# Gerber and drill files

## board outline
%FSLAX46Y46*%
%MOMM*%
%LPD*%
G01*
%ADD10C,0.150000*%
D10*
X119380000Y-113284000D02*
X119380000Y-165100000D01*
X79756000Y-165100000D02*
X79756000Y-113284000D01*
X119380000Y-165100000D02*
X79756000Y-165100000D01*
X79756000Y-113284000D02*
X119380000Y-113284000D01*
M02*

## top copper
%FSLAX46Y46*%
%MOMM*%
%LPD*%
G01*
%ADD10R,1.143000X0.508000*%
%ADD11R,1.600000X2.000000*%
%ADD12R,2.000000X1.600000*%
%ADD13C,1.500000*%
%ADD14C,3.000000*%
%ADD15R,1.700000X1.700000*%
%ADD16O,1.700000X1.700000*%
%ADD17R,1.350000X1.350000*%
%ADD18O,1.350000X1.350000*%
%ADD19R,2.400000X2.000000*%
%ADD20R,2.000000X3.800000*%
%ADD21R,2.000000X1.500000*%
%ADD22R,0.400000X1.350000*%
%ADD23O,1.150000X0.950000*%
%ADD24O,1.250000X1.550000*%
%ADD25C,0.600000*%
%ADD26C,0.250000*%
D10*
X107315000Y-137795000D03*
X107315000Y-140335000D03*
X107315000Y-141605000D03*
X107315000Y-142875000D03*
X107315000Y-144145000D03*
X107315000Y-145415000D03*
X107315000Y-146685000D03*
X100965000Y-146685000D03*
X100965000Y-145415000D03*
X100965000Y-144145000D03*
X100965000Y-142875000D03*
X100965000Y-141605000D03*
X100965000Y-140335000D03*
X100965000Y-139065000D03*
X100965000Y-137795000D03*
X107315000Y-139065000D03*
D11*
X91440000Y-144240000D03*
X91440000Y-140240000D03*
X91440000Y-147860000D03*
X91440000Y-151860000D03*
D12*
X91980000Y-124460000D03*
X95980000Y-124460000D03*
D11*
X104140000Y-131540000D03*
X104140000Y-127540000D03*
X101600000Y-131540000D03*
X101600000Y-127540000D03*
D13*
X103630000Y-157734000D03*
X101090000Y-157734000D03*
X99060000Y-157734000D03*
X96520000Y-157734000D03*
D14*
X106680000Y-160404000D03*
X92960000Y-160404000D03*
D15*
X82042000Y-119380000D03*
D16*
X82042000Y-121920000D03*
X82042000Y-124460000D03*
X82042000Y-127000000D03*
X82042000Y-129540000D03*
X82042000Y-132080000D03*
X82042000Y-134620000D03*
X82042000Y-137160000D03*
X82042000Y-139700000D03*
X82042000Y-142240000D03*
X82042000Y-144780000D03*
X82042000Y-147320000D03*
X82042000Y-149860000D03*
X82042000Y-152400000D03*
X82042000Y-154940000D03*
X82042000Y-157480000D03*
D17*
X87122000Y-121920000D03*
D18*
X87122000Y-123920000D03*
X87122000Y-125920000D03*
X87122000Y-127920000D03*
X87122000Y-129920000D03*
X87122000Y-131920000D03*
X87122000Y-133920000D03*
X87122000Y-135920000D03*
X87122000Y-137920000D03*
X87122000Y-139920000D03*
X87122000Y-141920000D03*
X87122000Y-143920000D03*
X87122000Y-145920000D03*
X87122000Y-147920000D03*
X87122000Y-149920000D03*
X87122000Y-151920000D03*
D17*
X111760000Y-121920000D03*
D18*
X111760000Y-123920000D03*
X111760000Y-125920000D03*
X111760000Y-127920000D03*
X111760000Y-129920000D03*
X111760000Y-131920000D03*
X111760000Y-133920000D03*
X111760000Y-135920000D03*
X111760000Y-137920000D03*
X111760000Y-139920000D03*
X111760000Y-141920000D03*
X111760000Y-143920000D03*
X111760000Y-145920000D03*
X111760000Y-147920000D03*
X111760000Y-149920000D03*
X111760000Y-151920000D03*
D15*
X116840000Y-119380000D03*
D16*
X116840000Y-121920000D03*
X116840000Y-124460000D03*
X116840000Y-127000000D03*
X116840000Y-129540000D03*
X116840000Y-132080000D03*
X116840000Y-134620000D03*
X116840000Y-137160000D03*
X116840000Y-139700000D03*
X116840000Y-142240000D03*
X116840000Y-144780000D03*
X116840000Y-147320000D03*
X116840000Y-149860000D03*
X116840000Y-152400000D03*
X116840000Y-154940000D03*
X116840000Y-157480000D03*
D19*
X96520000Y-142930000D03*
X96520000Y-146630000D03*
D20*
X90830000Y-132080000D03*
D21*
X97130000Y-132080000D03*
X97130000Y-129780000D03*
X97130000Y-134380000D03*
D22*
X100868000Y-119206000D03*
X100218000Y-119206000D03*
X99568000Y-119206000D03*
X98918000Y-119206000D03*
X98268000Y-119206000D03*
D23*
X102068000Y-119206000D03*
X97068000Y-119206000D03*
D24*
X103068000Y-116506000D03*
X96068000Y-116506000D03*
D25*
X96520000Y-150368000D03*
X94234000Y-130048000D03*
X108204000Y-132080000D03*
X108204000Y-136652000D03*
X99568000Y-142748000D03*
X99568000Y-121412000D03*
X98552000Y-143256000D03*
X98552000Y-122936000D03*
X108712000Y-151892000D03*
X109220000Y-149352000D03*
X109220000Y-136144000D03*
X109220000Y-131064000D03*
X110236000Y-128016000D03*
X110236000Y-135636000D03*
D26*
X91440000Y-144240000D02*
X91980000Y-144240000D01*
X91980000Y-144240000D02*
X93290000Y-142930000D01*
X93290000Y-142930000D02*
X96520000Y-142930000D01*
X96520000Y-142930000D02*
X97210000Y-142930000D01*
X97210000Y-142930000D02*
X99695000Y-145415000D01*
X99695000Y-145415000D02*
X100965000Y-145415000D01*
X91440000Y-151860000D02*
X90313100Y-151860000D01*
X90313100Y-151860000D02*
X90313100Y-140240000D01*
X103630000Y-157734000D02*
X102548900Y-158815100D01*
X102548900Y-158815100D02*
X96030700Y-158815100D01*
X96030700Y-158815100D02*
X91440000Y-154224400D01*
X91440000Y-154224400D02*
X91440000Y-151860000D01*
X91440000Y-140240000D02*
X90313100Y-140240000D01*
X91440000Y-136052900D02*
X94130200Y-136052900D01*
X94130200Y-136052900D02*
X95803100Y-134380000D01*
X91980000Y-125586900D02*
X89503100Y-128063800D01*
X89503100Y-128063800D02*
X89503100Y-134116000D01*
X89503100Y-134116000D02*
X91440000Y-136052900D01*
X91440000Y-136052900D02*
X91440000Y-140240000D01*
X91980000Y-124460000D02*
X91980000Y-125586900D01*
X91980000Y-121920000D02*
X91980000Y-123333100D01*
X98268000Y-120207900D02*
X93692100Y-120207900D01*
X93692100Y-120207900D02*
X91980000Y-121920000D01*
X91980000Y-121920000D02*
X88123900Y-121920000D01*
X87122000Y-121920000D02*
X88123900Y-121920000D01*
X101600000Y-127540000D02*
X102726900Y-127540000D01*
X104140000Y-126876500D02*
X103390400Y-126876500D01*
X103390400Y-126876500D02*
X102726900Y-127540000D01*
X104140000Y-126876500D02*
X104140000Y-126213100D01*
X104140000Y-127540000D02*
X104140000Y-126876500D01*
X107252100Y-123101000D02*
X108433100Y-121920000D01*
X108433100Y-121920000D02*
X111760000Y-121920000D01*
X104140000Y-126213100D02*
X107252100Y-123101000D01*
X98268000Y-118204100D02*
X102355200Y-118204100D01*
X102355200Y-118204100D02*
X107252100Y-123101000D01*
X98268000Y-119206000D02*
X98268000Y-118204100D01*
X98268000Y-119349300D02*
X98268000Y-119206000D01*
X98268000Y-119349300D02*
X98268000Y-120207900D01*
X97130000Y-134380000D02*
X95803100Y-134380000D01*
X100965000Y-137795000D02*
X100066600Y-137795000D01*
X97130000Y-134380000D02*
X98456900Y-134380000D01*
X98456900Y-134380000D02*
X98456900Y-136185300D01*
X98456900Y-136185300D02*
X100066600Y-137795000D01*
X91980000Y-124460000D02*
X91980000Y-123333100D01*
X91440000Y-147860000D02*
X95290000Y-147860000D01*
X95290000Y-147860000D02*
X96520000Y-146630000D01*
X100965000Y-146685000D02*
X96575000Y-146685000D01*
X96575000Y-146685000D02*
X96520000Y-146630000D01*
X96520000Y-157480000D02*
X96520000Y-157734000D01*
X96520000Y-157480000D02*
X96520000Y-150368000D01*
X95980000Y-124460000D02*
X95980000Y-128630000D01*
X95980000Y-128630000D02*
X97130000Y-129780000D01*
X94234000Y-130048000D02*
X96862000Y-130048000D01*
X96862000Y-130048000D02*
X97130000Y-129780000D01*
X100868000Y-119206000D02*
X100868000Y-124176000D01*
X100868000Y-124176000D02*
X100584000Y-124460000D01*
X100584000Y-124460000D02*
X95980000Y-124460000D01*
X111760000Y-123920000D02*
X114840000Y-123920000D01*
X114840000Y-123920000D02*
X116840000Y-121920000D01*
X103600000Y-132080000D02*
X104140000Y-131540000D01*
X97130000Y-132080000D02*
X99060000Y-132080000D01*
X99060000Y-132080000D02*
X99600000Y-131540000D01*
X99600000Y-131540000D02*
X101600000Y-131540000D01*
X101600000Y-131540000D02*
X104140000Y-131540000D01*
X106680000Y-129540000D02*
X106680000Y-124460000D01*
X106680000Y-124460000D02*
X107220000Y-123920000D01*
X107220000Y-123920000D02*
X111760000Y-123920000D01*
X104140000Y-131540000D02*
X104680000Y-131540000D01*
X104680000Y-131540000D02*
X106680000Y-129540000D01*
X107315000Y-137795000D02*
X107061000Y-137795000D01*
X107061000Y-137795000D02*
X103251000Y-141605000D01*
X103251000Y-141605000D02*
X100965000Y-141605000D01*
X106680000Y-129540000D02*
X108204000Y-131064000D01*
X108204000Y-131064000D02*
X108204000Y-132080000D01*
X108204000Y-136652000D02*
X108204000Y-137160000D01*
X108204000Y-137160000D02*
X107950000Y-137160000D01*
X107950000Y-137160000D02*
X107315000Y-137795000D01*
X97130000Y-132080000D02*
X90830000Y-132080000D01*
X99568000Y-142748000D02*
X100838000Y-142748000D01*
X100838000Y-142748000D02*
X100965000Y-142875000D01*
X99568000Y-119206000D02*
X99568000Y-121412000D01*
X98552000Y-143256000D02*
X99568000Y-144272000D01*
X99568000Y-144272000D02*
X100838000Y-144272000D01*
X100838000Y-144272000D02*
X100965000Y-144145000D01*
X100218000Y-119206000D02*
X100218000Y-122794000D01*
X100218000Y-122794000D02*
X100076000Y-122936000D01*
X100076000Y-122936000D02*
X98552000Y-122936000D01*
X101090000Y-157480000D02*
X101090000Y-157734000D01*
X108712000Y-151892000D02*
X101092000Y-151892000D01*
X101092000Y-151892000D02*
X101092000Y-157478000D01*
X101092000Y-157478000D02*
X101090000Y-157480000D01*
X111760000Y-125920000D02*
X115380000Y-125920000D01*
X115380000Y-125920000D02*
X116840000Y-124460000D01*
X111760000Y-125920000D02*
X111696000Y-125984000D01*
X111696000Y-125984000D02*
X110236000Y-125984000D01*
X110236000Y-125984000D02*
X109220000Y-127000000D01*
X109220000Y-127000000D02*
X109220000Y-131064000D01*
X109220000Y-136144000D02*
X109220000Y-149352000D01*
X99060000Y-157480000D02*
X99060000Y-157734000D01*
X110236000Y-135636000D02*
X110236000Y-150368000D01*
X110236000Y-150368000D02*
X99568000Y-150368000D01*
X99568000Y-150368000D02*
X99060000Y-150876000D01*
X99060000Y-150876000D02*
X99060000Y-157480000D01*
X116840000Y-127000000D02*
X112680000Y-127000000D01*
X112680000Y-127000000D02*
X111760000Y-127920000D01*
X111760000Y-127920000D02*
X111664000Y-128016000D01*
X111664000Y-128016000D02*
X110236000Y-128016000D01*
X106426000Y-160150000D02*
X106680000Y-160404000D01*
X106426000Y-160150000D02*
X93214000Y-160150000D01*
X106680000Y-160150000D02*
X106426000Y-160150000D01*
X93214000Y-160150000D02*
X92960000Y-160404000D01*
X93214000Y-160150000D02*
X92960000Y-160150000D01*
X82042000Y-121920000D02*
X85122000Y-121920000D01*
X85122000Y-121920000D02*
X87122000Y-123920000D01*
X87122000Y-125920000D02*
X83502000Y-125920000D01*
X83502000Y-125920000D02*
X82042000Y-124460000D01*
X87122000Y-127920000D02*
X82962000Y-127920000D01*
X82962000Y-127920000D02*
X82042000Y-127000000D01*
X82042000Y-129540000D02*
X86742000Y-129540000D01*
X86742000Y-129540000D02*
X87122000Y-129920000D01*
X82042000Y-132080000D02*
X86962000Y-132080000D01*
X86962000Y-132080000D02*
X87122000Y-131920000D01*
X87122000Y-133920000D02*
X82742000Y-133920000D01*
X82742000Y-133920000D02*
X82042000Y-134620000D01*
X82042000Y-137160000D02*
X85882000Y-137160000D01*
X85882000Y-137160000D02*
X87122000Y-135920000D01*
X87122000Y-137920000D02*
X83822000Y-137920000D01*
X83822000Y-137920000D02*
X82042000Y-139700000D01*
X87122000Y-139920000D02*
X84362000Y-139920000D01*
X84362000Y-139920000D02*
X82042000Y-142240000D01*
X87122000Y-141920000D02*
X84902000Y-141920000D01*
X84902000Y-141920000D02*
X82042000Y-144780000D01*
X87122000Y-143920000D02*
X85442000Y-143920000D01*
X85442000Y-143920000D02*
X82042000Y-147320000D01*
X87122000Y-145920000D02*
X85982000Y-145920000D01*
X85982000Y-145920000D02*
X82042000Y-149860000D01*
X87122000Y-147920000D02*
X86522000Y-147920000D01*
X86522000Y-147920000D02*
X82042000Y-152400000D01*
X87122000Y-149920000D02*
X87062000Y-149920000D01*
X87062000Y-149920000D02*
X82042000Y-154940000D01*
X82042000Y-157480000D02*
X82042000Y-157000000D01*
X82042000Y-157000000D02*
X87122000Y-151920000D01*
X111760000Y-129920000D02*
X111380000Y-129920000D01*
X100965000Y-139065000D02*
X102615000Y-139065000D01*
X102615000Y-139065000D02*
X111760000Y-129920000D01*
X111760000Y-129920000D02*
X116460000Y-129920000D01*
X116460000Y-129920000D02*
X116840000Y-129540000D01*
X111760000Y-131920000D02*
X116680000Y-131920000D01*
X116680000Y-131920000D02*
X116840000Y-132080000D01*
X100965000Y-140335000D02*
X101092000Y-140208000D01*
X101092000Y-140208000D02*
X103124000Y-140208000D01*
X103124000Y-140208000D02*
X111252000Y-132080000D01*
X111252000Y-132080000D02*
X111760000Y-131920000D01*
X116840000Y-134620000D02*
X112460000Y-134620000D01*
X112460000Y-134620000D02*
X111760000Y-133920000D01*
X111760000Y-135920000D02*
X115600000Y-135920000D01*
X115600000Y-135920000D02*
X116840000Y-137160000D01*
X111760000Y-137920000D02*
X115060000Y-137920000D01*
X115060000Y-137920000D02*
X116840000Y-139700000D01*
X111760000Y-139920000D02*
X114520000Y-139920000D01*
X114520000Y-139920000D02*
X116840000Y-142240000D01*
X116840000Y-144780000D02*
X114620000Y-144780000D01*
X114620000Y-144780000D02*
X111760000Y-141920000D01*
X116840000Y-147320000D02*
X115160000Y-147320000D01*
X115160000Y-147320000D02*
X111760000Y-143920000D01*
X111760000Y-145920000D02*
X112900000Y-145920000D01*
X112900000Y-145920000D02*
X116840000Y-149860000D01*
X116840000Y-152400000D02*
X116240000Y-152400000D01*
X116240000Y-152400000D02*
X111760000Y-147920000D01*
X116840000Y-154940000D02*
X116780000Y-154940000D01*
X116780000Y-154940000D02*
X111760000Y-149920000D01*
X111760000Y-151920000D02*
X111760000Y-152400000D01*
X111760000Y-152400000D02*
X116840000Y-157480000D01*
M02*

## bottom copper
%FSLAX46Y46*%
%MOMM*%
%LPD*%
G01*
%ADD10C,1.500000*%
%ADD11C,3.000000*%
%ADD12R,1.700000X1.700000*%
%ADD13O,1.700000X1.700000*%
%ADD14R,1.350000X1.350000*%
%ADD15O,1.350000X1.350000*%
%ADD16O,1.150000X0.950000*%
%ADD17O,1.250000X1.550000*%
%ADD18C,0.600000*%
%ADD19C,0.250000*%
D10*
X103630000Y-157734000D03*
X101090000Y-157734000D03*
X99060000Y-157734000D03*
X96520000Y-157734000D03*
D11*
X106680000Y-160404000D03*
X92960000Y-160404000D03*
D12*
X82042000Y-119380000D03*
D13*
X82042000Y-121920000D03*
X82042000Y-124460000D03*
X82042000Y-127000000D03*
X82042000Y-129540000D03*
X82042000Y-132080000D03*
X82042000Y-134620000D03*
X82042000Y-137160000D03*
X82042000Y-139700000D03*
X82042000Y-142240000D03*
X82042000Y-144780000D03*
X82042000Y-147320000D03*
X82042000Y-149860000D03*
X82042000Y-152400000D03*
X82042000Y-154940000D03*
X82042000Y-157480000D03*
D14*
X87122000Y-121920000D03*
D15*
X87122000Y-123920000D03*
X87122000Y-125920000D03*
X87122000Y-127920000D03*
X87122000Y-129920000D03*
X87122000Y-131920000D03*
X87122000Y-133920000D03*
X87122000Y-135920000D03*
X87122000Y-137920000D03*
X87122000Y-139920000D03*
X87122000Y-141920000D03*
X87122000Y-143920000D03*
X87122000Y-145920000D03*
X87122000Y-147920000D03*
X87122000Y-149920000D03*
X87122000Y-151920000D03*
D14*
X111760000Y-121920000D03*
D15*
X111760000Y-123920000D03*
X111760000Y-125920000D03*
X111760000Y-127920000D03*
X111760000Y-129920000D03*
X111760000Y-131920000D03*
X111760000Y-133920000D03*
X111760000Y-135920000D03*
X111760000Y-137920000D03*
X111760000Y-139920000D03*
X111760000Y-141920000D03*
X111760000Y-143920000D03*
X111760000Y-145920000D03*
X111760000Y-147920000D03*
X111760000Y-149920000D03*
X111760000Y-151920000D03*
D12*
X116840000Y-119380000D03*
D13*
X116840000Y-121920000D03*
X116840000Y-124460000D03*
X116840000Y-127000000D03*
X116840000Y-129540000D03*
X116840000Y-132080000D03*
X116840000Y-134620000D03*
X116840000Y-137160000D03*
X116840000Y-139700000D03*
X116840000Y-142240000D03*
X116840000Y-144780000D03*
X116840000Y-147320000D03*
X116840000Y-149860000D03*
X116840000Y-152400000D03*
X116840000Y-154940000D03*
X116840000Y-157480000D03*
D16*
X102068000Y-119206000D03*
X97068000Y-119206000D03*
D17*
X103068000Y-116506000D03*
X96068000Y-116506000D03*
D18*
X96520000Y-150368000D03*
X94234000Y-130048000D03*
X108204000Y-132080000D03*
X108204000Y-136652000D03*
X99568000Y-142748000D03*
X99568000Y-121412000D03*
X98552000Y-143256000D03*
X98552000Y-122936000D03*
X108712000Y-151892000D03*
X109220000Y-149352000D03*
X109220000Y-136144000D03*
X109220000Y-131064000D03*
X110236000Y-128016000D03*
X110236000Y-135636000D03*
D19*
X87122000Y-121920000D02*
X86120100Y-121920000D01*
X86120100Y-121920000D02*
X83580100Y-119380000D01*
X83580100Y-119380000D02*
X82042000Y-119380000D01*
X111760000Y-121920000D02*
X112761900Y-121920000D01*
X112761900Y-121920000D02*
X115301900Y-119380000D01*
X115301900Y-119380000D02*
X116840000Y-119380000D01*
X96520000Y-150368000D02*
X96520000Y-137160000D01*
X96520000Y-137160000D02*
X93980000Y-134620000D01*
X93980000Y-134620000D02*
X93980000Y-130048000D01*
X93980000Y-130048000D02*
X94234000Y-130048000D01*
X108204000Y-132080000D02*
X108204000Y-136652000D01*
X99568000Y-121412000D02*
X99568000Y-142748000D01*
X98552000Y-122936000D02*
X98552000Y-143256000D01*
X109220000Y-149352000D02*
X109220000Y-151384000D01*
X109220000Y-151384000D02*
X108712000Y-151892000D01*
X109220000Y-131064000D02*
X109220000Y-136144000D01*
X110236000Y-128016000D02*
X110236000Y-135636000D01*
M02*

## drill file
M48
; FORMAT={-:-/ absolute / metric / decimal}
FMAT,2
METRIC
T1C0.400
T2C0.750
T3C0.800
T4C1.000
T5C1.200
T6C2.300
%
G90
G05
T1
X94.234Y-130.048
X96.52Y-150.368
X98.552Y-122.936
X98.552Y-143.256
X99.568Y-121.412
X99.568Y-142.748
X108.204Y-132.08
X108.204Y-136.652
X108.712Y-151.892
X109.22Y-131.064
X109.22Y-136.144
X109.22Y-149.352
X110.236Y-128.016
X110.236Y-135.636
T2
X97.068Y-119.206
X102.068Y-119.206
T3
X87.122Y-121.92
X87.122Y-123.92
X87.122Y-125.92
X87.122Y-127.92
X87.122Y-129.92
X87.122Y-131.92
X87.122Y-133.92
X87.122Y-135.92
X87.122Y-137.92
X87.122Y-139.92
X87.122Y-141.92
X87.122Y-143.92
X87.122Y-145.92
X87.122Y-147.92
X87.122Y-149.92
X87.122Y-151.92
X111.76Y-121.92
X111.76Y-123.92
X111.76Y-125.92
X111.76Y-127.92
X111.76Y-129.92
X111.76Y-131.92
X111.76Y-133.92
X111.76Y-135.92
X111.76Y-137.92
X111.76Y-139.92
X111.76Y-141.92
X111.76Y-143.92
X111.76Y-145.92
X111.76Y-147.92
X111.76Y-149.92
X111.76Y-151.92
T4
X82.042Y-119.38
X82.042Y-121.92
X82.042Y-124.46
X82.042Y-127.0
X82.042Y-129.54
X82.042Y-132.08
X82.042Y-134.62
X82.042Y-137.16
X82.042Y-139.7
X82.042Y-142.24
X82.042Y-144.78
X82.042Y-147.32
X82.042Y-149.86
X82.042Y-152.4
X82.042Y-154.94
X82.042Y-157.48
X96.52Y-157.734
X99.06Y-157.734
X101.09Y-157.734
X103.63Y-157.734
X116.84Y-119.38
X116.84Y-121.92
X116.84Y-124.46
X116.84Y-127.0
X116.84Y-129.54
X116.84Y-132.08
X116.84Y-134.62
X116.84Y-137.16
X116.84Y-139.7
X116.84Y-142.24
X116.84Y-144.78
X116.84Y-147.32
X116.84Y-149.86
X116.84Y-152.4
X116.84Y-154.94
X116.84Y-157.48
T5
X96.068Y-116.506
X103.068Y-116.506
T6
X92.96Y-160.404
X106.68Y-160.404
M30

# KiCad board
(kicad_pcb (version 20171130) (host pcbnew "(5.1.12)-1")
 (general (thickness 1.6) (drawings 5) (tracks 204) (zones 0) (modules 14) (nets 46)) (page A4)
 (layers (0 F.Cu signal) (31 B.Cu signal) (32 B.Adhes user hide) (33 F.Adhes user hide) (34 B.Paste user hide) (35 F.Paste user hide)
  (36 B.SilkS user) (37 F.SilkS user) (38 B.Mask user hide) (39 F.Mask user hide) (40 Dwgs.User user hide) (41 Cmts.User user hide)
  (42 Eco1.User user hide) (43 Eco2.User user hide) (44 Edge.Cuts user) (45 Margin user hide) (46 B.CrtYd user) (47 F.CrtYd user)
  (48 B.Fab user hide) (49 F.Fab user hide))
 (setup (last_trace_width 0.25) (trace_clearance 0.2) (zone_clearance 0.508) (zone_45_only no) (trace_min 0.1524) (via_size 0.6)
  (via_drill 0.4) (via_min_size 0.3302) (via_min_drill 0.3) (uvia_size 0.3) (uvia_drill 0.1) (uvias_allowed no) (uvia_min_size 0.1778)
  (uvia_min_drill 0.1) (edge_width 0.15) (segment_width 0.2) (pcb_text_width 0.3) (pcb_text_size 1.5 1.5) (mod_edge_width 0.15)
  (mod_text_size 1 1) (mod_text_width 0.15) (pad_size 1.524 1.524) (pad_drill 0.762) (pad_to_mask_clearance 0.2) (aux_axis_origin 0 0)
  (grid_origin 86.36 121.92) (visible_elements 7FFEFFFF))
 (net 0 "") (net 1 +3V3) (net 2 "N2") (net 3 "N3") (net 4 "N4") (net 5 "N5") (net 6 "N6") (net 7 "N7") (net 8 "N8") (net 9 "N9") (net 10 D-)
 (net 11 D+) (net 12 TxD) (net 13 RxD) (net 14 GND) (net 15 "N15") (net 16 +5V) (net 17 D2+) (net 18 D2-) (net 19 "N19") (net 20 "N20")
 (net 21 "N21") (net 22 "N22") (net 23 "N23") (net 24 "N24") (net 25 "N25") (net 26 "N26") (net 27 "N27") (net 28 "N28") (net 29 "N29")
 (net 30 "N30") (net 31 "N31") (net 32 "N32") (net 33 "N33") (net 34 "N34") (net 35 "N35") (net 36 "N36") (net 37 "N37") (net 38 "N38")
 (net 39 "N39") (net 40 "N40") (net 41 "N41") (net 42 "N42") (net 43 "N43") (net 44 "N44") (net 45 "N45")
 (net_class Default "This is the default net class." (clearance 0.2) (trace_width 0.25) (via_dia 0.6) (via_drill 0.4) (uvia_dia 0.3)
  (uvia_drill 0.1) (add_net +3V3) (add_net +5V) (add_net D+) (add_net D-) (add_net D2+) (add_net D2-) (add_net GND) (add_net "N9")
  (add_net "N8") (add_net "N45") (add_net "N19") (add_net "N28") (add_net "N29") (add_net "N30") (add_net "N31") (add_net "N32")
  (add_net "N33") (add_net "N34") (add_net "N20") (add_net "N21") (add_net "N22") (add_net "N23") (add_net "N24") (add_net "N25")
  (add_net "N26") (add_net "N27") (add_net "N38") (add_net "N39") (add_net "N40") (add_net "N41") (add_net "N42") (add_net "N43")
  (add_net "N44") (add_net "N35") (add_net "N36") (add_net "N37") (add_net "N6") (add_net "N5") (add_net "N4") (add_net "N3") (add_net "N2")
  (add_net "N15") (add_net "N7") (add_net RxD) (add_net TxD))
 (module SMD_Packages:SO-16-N (layer F.Cu) (at 104.14 142.24 270)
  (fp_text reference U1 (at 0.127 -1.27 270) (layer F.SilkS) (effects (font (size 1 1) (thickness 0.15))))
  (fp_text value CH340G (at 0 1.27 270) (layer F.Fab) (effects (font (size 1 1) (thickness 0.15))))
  (pad 16 smd rect (at -4.445 -3.175 270) (size 0.508 1.143) (layers F.Cu F.Paste F.Mask) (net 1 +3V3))
  (pad 14 smd rect (at -1.905 -3.175 270) (size 0.508 1.143) (layers F.Cu F.Paste F.Mask) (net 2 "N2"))
  (pad 13 smd rect (at -0.635 -3.175 270) (size 0.508 1.143) (layers F.Cu F.Paste F.Mask) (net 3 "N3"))
  (pad 12 smd rect (at 0.635 -3.175 270) (size 0.508 1.143) (layers F.Cu F.Paste F.Mask) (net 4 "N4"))
  (pad 11 smd rect (at 1.905 -3.175 270) (size 0.508 1.143) (layers F.Cu F.Paste F.Mask) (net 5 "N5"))
  (pad 10 smd rect (at 3.175 -3.175 270) (size 0.508 1.143) (layers F.Cu F.Paste F.Mask) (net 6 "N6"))
  (pad 9 smd rect (at 4.445 -3.175 270) (size 0.508 1.143) (layers F.Cu F.Paste F.Mask) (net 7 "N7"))
  (pad 8 smd rect (at 4.445 3.175 270) (size 0.508 1.143) (layers F.Cu F.Paste F.Mask) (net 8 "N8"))
  (pad 7 smd rect (at 3.175 3.175 270) (size 0.508 1.143) (layers F.Cu F.Paste F.Mask) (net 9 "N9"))
  (pad 6 smd rect (at 1.905 3.175 270) (size 0.508 1.143) (layers F.Cu F.Paste F.Mask) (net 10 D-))
  (pad 5 smd rect (at 0.635 3.175 270) (size 0.508 1.143) (layers F.Cu F.Paste F.Mask) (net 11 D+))
  (pad 4 smd rect (at -0.635 3.175 270) (size 0.508 1.143) (layers F.Cu F.Paste F.Mask) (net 1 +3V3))
  (pad 3 smd rect (at -1.905 3.175 270) (size 0.508 1.143) (layers F.Cu F.Paste F.Mask) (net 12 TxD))
  (pad 2 smd rect (at -3.175 3.175 270) (size 0.508 1.143) (layers F.Cu F.Paste F.Mask) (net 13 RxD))
  (pad 1 smd rect (at -4.445 3.175 270) (size 0.508 1.143) (layers F.Cu F.Paste F.Mask) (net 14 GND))
  (pad 15 smd rect (at -3.175 -3.175 270) (size 0.508 1.143) (layers F.Cu F.Paste F.Mask) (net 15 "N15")))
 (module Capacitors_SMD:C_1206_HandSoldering (layer F.Cu) (at 91.44 142.24 90)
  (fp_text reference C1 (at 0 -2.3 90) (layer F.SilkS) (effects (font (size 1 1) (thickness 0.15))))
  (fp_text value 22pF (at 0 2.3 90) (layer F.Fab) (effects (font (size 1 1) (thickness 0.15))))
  (pad 1 smd rect (at -2 0 90) (size 2 1.6) (layers F.Cu F.Paste F.Mask) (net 9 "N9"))
  (pad 2 smd rect (at 2 0 90) (size 2 1.6) (layers F.Cu F.Paste F.Mask) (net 14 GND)))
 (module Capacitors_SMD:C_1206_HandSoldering (layer F.Cu) (at 91.44 149.86 270)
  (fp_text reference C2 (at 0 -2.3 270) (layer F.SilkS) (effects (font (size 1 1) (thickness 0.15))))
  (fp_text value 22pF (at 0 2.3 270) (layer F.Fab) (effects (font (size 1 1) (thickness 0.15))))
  (pad 1 smd rect (at -2 0 270) (size 2 1.6) (layers F.Cu F.Paste F.Mask) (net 8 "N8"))
  (pad 2 smd rect (at 2 0 270) (size 2 1.6) (layers F.Cu F.Paste F.Mask) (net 14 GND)))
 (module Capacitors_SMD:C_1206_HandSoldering (layer F.Cu) (at 93.98 124.46)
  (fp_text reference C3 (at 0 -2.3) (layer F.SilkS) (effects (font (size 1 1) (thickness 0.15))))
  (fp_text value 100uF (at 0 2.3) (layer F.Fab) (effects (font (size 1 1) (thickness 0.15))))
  (pad 1 smd rect (at -2 0) (size 2 1.6) (layers F.Cu F.Paste F.Mask) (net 14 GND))
  (pad 2 smd rect (at 2 0) (size 2 1.6) (layers F.Cu F.Paste F.Mask) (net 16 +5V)))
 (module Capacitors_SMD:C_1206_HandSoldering (layer F.Cu) (at 104.14 129.54 90)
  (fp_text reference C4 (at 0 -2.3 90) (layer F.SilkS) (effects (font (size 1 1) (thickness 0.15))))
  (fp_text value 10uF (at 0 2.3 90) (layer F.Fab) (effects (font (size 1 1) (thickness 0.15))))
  (pad 1 smd rect (at -2 0 90) (size 2 1.6) (layers F.Cu F.Paste F.Mask) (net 1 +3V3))
  (pad 2 smd rect (at 2 0 90) (size 2 1.6) (layers F.Cu F.Paste F.Mask) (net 14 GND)))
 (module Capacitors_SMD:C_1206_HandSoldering (layer F.Cu) (at 101.6 129.54 90)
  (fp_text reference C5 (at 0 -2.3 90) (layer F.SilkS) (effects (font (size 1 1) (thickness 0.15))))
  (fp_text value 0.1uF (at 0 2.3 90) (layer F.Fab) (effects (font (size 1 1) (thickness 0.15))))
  (pad 1 smd rect (at -2 0 90) (size 2 1.6) (layers F.Cu F.Paste F.Mask) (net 1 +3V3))
  (pad 2 smd rect (at 2 0 90) (size 2 1.6) (layers F.Cu F.Paste F.Mask) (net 14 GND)))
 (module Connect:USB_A (layer F.Cu) (at 96.52 157.734)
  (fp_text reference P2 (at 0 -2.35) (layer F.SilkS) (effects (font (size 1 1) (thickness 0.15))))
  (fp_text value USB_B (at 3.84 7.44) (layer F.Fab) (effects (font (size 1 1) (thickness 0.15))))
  (pad 4 thru_hole circle (at 7.11 0 270) (size 1.5 1.5) (drill 1) (layers *.Cu *.Mask) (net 14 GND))
  (pad 3 thru_hole circle (at 4.57 0 270) (size 1.5 1.5) (drill 1) (layers *.Cu *.Mask) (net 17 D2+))
  (pad 2 thru_hole circle (at 2.54 0 270) (size 1.5 1.5) (drill 1) (layers *.Cu *.Mask) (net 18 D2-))
  (pad 1 thru_hole circle (at 0 0 270) (size 1.5 1.5) (drill 1) (layers *.Cu *.Mask) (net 16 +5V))
  (pad 5 thru_hole circle (at 10.16 2.67 270) (size 3 3) (drill 2.3) (layers *.Cu *.Mask) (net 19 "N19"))
  (pad 5 thru_hole circle (at -3.56 2.67 270) (size 3 3) (drill 2.3) (layers *.Cu *.Mask) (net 19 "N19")))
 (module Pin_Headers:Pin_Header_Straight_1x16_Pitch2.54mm (layer F.Cu) (at 82.042 119.38)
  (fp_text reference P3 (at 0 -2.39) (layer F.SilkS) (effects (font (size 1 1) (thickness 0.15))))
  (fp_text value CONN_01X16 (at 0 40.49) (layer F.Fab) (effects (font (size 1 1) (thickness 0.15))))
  (pad 1 thru_hole rect (at 0 0) (size 1.7 1.7) (drill 1) (layers *.Cu *.Mask) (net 14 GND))
  (pad 2 thru_hole oval (at 0 2.54) (size 1.7 1.7) (drill 1) (layers *.Cu *.Mask) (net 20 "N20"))
  (pad 3 thru_hole oval (at 0 5.08) (size 1.7 1.7) (drill 1) (layers *.Cu *.Mask) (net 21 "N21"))
  (pad 4 thru_hole oval (at 0 7.62) (size 1.7 1.7) (drill 1) (layers *.Cu *.Mask) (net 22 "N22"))
  (pad 5 thru_hole oval (at 0 10.16) (size 1.7 1.7) (drill 1) (layers *.Cu *.Mask) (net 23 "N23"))
  (pad 6 thru_hole oval (at 0 12.7) (size 1.7 1.7) (drill 1) (layers *.Cu *.Mask) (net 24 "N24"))
  (pad 7 thru_hole oval (at 0 15.24) (size 1.7 1.7) (drill 1) (layers *.Cu *.Mask) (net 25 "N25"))
  (pad 8 thru_hole oval (at 0 17.78) (size 1.7 1.7) (drill 1) (layers *.Cu *.Mask) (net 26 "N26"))
  (pad 9 thru_hole oval (at 0 20.32) (size 1.7 1.7) (drill 1) (layers *.Cu *.Mask) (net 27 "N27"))
  (pad 10 thru_hole oval (at 0 22.86) (size 1.7 1.7) (drill 1) (layers *.Cu *.Mask) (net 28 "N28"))
  (pad 11 thru_hole oval (at 0 25.4) (size 1.7 1.7) (drill 1) (layers *.Cu *.Mask) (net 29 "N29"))
  (pad 12 thru_hole oval (at 0 27.94) (size 1.7 1.7) (drill 1) (layers *.Cu *.Mask) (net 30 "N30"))
  (pad 13 thru_hole oval (at 0 30.48) (size 1.7 1.7) (drill 1) (layers *.Cu *.Mask) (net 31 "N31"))
  (pad 14 thru_hole oval (at 0 33.02) (size 1.7 1.7) (drill 1) (layers *.Cu *.Mask) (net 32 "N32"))
  (pad 15 thru_hole oval (at 0 35.56) (size 1.7 1.7) (drill 1) (layers *.Cu *.Mask) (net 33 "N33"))
  (pad 16 thru_hole oval (at 0 38.1) (size 1.7 1.7) (drill 1) (layers *.Cu *.Mask) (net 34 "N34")))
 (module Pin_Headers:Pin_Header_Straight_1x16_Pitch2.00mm (layer F.Cu) (at 87.122 121.92)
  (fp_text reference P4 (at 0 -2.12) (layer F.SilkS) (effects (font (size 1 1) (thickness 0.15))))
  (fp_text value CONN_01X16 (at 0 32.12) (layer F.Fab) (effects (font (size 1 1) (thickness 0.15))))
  (pad 1 thru_hole rect (at 0 0) (size 1.35 1.35) (drill 0.8) (layers *.Cu *.Mask) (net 14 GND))
  (pad 2 thru_hole oval (at 0 2) (size 1.35 1.35) (drill 0.8) (layers *.Cu *.Mask) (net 20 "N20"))
  (pad 3 thru_hole oval (at 0 4) (size 1.35 1.35) (drill 0.8) (layers *.Cu *.Mask) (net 21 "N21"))
  (pad 4 thru_hole oval (at 0 6) (size 1.35 1.35) (drill 0.8) (layers *.Cu *.Mask) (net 22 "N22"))
  (pad 5 thru_hole oval (at 0 8) (size 1.35 1.35) (drill 0.8) (layers *.Cu *.Mask) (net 23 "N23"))
  (pad 6 thru_hole oval (at 0 10) (size 1.35 1.35) (drill 0.8) (layers *.Cu *.Mask) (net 24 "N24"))
  (pad 7 thru_hole oval (at 0 12) (size 1.35 1.35) (drill 0.8) (layers *.Cu *.Mask) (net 25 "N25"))
  (pad 8 thru_hole oval (at 0 14) (size 1.35 1.35) (drill 0.8) (layers *.Cu *.Mask) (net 26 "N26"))
  (pad 9 thru_hole oval (at 0 16) (size 1.35 1.35) (drill 0.8) (layers *.Cu *.Mask) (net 27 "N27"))
  (pad 10 thru_hole oval (at 0 18) (size 1.35 1.35) (drill 0.8) (layers *.Cu *.Mask) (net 28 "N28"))
  (pad 11 thru_hole oval (at 0 20) (size 1.35 1.35) (drill 0.8) (layers *.Cu *.Mask) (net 29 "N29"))
  (pad 12 thru_hole oval (at 0 22) (size 1.35 1.35) (drill 0.8) (layers *.Cu *.Mask) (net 30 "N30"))
  (pad 13 thru_hole oval (at 0 24) (size 1.35 1.35) (drill 0.8) (layers *.Cu *.Mask) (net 31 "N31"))
  (pad 14 thru_hole oval (at 0 26) (size 1.35 1.35) (drill 0.8) (layers *.Cu *.Mask) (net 32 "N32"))
  (pad 15 thru_hole oval (at 0 28) (size 1.35 1.35) (drill 0.8) (layers *.Cu *.Mask) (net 33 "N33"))
  (pad 16 thru_hole oval (at 0 30) (size 1.35 1.35) (drill 0.8) (layers *.Cu *.Mask) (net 34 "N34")))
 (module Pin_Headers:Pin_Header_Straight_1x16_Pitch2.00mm (layer F.Cu) (at 111.76 121.92)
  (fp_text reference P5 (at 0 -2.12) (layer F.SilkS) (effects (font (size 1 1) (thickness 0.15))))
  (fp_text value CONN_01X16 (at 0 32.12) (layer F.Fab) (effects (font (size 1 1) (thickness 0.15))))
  (pad 1 thru_hole rect (at 0 0) (size 1.35 1.35) (drill 0.8) (layers *.Cu *.Mask) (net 14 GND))
  (pad 2 thru_hole oval (at 0 2) (size 1.35 1.35) (drill 0.8) (layers *.Cu *.Mask) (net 1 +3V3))
  (pad 3 thru_hole oval (at 0 4) (size 1.35 1.35) (drill 0.8) (layers *.Cu *.Mask) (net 17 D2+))
  (pad 4 thru_hole oval (at 0 6) (size 1.35 1.35) (drill 0.8) (layers *.Cu *.Mask) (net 18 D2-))
  (pad 5 thru_hole oval (at 0 8) (size 1.35 1.35) (drill 0.8) (layers *.Cu *.Mask) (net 13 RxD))
  (pad 6 thru_hole oval (at 0 10) (size 1.35 1.35) (drill 0.8) (layers *.Cu *.Mask) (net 12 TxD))
  (pad 7 thru_hole oval (at 0 12) (size 1.35 1.35) (drill 0.8) (layers *.Cu *.Mask) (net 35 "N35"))
  (pad 8 thru_hole oval (at 0 14) (size 1.35 1.35) (drill 0.8) (layers *.Cu *.Mask) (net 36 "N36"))
  (pad 9 thru_hole oval (at 0 16) (size 1.35 1.35) (drill 0.8) (layers *.Cu *.Mask) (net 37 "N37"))
  (pad 10 thru_hole oval (at 0 18) (size 1.35 1.35) (drill 0.8) (layers *.Cu *.Mask) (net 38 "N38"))
  (pad 11 thru_hole oval (at 0 20) (size 1.35 1.35) (drill 0.8) (layers *.Cu *.Mask) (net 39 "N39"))
  (pad 12 thru_hole oval (at 0 22) (size 1.35 1.35) (drill 0.8) (layers *.Cu *.Mask) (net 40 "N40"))
  (pad 13 thru_hole oval (at 0 24) (size 1.35 1.35) (drill 0.8) (layers *.Cu *.Mask) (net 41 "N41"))
  (pad 14 thru_hole oval (at 0 26) (size 1.35 1.35) (drill 0.8) (layers *.Cu *.Mask) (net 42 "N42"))
  (pad 15 thru_hole oval (at 0 28) (size 1.35 1.35) (drill 0.8) (layers *.Cu *.Mask) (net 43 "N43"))
  (pad 16 thru_hole oval (at 0 30) (size 1.35 1.35) (drill 0.8) (layers *.Cu *.Mask) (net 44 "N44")))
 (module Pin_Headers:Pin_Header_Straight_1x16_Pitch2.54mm (layer F.Cu) (at 116.84 119.38)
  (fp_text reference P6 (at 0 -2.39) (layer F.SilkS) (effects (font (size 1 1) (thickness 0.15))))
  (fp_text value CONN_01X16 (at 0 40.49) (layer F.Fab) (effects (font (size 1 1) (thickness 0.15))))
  (pad 1 thru_hole rect (at 0 0) (size 1.7 1.7) (drill 1) (layers *.Cu *.Mask) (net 14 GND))
  (pad 2 thru_hole oval (at 0 2.54) (size 1.7 1.7) (drill 1) (layers *.Cu *.Mask) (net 1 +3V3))
  (pad 3 thru_hole oval (at 0 5.08) (size 1.7 1.7) (drill 1) (layers *.Cu *.Mask) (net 17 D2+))
  (pad 4 thru_hole oval (at 0 7.62) (size 1.7 1.7) (drill 1) (layers *.Cu *.Mask) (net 18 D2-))
  (pad 5 thru_hole oval (at 0 10.16) (size 1.7 1.7) (drill 1) (layers *.Cu *.Mask) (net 13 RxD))
  (pad 6 thru_hole oval (at 0 12.7) (size 1.7 1.7) (drill 1) (layers *.Cu *.Mask) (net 12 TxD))
  (pad 7 thru_hole oval (at 0 15.24) (size 1.7 1.7) (drill 1) (layers *.Cu *.Mask) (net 35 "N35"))
  (pad 8 thru_hole oval (at 0 17.78) (size 1.7 1.7) (drill 1) (layers *.Cu *.Mask) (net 36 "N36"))
  (pad 9 thru_hole oval (at 0 20.32) (size 1.7 1.7) (drill 1) (layers *.Cu *.Mask) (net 37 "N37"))
  (pad 10 thru_hole oval (at 0 22.86) (size 1.7 1.7) (drill 1) (layers *.Cu *.Mask) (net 38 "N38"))
  (pad 11 thru_hole oval (at 0 25.4) (size 1.7 1.7) (drill 1) (layers *.Cu *.Mask) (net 39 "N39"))
  (pad 12 thru_hole oval (at 0 27.94) (size 1.7 1.7) (drill 1) (layers *.Cu *.Mask) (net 40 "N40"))
  (pad 13 thru_hole oval (at 0 30.48) (size 1.7 1.7) (drill 1) (layers *.Cu *.Mask) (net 41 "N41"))
  (pad 14 thru_hole oval (at 0 33.02) (size 1.7 1.7) (drill 1) (layers *.Cu *.Mask) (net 42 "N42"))
  (pad 15 thru_hole oval (at 0 35.56) (size 1.7 1.7) (drill 1) (layers *.Cu *.Mask) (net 43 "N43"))
  (pad 16 thru_hole oval (at 0 38.1) (size 1.7 1.7) (drill 1) (layers *.Cu *.Mask) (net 44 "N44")))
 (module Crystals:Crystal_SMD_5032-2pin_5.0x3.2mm (layer F.Cu) (at 96.52 144.78 270)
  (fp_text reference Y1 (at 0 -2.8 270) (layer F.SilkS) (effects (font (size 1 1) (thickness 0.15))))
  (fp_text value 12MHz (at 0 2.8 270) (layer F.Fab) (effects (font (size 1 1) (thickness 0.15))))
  (pad 1 smd rect (at -1.85 0 270) (size 2 2.4) (layers F.Cu F.Mask) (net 9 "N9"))
  (pad 2 smd rect (at 1.85 0 270) (size 2 2.4) (layers F.Cu F.Mask) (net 8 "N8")))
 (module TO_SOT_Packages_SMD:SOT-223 (layer F.Cu) (at 93.98 132.08 180)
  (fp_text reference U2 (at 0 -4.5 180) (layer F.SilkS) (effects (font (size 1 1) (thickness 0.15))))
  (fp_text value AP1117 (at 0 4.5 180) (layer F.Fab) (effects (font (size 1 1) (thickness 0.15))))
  (pad 4 smd rect (at 3.15 0 180) (size 2 3.8) (layers F.Cu F.Paste F.Mask) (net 1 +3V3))
  (pad 2 smd rect (at -3.15 0 180) (size 2 1.5) (layers F.Cu F.Paste F.Mask) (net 1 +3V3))
  (pad 3 smd rect (at -3.15 2.3 180) (size 2 1.5) (layers F.Cu F.Paste F.Mask) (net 16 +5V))
  (pad 1 smd rect (at -3.15 -2.3 180) (size 2 1.5) (layers F.Cu F.Paste F.Mask) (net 14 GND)))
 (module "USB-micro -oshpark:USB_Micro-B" (layer F.Cu) (at 99.568 117.856 180)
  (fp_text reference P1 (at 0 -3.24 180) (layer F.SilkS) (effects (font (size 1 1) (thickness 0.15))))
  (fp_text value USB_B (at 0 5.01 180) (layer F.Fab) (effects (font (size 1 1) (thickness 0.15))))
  (pad 1 smd rect (at -1.3 -1.35 270) (size 1.35 0.4) (layers F.Cu F.Paste F.Mask) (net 16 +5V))
  (pad 2 smd rect (at -0.65 -1.35 270) (size 1.35 0.4) (layers F.Cu F.Paste F.Mask) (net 10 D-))
  (pad 3 smd rect (at 0 -1.35 270) (size 1.35 0.4) (layers F.Cu F.Paste F.Mask) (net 11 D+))
  (pad 4 smd rect (at 0.65 -1.35 270) (size 1.35 0.4) (layers F.Cu F.Paste F.Mask) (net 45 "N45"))
  (pad 5 smd rect (at 1.3 -1.35 270) (size 1.35 0.4) (layers F.Cu F.Paste F.Mask) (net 14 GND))
  (pad 6 thru_hole oval (at -2.5 -1.35 270) (size 0.95 1.15) (drill 0.75) (layers *.Cu *.Mask))
  (pad 6 thru_hole oval (at 2.5 -1.35 270) (size 0.95 1.15) (drill 0.75) (layers *.Cu *.Mask))
  (pad 6 thru_hole oval (at -3.5 1.35 270) (size 1.55 1.25) (drill 1.2) (layers *.Cu *.Mask))
  (pad 6 thru_hole oval (at 3.5 1.35 270) (size 1.55 1.25) (drill 1.2) (layers *.Cu *.Mask)))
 (gr_line (start 119.38 113.284) (end 119.38 165.1) (angle 90) (layer Edge.Cuts) (width 0.15))
 (gr_line (start 79.756 165.1) (end 79.756 113.284) (angle 90) (layer Edge.Cuts) (width 0.15))
 (gr_line (start 119.38 165.1) (end 79.756 165.1) (angle 90) (layer Edge.Cuts) (width 0.15))
 (gr_line (start 79.756 113.284) (end 119.38 113.284) (angle 90) (layer Edge.Cuts) (width 0.15))
 (segment (start 91.44 144.24) (end 91.98 144.24) (width 0.25) (layer F.Cu) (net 9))
 (segment (start 91.98 144.24) (end 93.29 142.93) (width 0.25) (layer F.Cu) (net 9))
 (segment (start 93.29 142.93) (end 96.52 142.93) (width 0.25) (layer F.Cu) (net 9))
 (segment (start 96.52 142.93) (end 97.21 142.93) (width 0.25) (layer F.Cu) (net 9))
 (segment (start 97.21 142.93) (end 99.695 145.415) (width 0.25) (layer F.Cu) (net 9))
 (segment (start 99.695 145.415) (end 100.965 145.415) (width 0.25) (layer F.Cu) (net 9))
 (segment (start 91.44 151.86) (end 90.3131 151.86) (width 0.25) (layer F.Cu) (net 14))
 (segment (start 90.3131 151.86) (end 90.3131 140.24) (width 0.25) (layer F.Cu) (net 14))
 (segment (start 103.63 157.734) (end 102.5489 158.8151) (width 0.25) (layer F.Cu) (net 14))
 (segment (start 102.5489 158.8151) (end 96.0307 158.8151) (width 0.25) (layer F.Cu) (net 14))
 (segment (start 96.0307 158.8151) (end 91.44 154.2244) (width 0.25) (layer F.Cu) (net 14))
 (segment (start 91.44 154.2244) (end 91.44 151.86) (width 0.25) (layer F.Cu) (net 14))
 (segment (start 91.44 140.24) (end 90.3131 140.24) (width 0.25) (layer F.Cu) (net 14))
 (segment (start 91.44 136.0529) (end 94.1302 136.0529) (width 0.25) (layer F.Cu) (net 14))
 (segment (start 94.1302 136.0529) (end 95.8031 134.38) (width 0.25) (layer F.Cu) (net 14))
 (segment (start 91.98 125.5869) (end 89.5031 128.0638) (width 0.25) (layer F.Cu) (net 14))
 (segment (start 89.5031 128.0638) (end 89.5031 134.116) (width 0.25) (layer F.Cu) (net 14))
 (segment (start 89.5031 134.116) (end 91.44 136.0529) (width 0.25) (layer F.Cu) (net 14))
 (segment (start 91.44 136.0529) (end 91.44 140.24) (width 0.25) (layer F.Cu) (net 14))
 (segment (start 91.98 124.46) (end 91.98 125.5869) (width 0.25) (layer F.Cu) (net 14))
 (segment (start 91.98 121.92) (end 91.98 123.3331) (width 0.25) (layer F.Cu) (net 14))
 (segment (start 98.268 120.2079) (end 93.6921 120.2079) (width 0.25) (layer F.Cu) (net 14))
 (segment (start 93.6921 120.2079) (end 91.98 121.92) (width 0.25) (layer F.Cu) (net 14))
 (segment (start 91.98 121.92) (end 88.1239 121.92) (width 0.25) (layer F.Cu) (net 14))
 (segment (start 87.122 121.92) (end 88.1239 121.92) (width 0.25) (layer F.Cu) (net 14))
 (segment (start 101.6 127.54) (end 102.7269 127.54) (width 0.25) (layer F.Cu) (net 14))
 (segment (start 104.14 126.8765) (end 103.3904 126.8765) (width 0.25) (layer F.Cu) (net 14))
 (segment (start 103.3904 126.8765) (end 102.7269 127.54) (width 0.25) (layer F.Cu) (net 14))
 (segment (start 104.14 126.8765) (end 104.14 126.2131) (width 0.25) (layer F.Cu) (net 14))
 (segment (start 104.14 127.54) (end 104.14 126.8765) (width 0.25) (layer F.Cu) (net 14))
 (segment (start 107.2521 123.101) (end 108.4331 121.92) (width 0.25) (layer F.Cu) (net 14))
 (segment (start 108.4331 121.92) (end 111.76 121.92) (width 0.25) (layer F.Cu) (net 14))
 (segment (start 104.14 126.2131) (end 107.2521 123.101) (width 0.25) (layer F.Cu) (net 14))
 (segment (start 98.268 118.2041) (end 102.3552 118.2041) (width 0.25) (layer F.Cu) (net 14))
 (segment (start 102.3552 118.2041) (end 107.2521 123.101) (width 0.25) (layer F.Cu) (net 14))
 (segment (start 98.268 119.206) (end 98.268 118.2041) (width 0.25) (layer F.Cu) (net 14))
 (segment (start 98.268 119.3493) (end 98.268 119.206) (width 0.25) (layer F.Cu) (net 14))
 (segment (start 98.268 119.3493) (end 98.268 120.2079) (width 0.25) (layer F.Cu) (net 14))
 (segment (start 97.13 134.38) (end 95.8031 134.38) (width 0.25) (layer F.Cu) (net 14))
 (segment (start 87.122 121.92) (end 86.1201 121.92) (width 0.25) (layer B.Cu) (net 14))
 (segment (start 86.1201 121.92) (end 83.5801 119.38) (width 0.25) (layer B.Cu) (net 14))
 (segment (start 83.5801 119.38) (end 82.042 119.38) (width 0.25) (layer B.Cu) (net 14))
 (segment (start 111.76 121.92) (end 112.7619 121.92) (width 0.25) (layer B.Cu) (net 14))
 (segment (start 112.7619 121.92) (end 115.3019 119.38) (width 0.25) (layer B.Cu) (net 14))
 (segment (start 115.3019 119.38) (end 116.84 119.38) (width 0.25) (layer B.Cu) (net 14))
 (segment (start 100.965 137.795) (end 100.0666 137.795) (width 0.25) (layer F.Cu) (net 14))
 (segment (start 97.13 134.38) (end 98.4569 134.38) (width 0.25) (layer F.Cu) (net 14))
 (segment (start 98.4569 134.38) (end 98.4569 136.1853) (width 0.25) (layer F.Cu) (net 14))
 (segment (start 98.4569 136.1853) (end 100.0666 137.795) (width 0.25) (layer F.Cu) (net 14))
 (segment (start 91.98 124.46) (end 91.98 123.3331) (width 0.25) (layer F.Cu) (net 14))
 (segment (start 91.44 147.86) (end 95.29 147.86) (width 0.25) (layer F.Cu) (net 8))
 (segment (start 95.29 147.86) (end 96.52 146.63) (width 0.25) (layer F.Cu) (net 8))
 (segment (start 100.965 146.685) (end 96.575 146.685) (width 0.25) (layer F.Cu) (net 8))
 (segment (start 96.575 146.685) (end 96.52 146.63) (width 0.25) (layer F.Cu) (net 8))
 (segment (start 96.52 157.48) (end 96.52 157.734) (width 0.25) (layer F.Cu) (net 16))
 (segment (start 96.52 157.48) (end 96.52 150.368) (width 0.25) (layer F.Cu) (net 16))
 (segment (start 95.98 124.46) (end 95.98 128.63) (width 0.25) (layer F.Cu) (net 16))
 (segment (start 95.98 128.63) (end 97.13 129.78) (width 0.25) (layer F.Cu) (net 16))
 (segment (start 94.234 130.048) (end 96.862 130.048) (width 0.25) (layer F.Cu) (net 16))
 (segment (start 96.862 130.048) (end 97.13 129.78) (width 0.25) (layer F.Cu) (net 16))
 (segment (start 96.52 150.368) (end 96.52 137.16) (width 0.25) (layer B.Cu) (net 16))
 (segment (start 96.52 137.16) (end 93.98 134.62) (width 0.25) (layer B.Cu) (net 16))
 (segment (start 93.98 134.62) (end 93.98 130.048) (width 0.25) (layer B.Cu) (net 16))
 (segment (start 93.98 130.048) (end 94.234 130.048) (width 0.25) (layer B.Cu) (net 16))
 (segment (start 100.868 119.206) (end 100.868 124.176) (width 0.25) (layer F.Cu) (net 16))
 (segment (start 100.868 124.176) (end 100.584 124.46) (width 0.25) (layer F.Cu) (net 16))
 (segment (start 100.584 124.46) (end 95.98 124.46) (width 0.25) (layer F.Cu) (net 16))
 (via (at 96.52 150.368) (size 0.6) (layers F.Cu B.Cu) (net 16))
 (via (at 94.234 130.048) (size 0.6) (layers F.Cu B.Cu) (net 16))
 (segment (start 111.76 123.92) (end 114.84 123.92) (width 0.25) (layer F.Cu) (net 1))
 (segment (start 114.84 123.92) (end 116.84 121.92) (width 0.25) (layer F.Cu) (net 1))
 (segment (start 103.6 132.08) (end 104.14 131.54) (width 0.25) (layer F.Cu) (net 1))
 (segment (start 97.13 132.08) (end 99.06 132.08) (width 0.25) (layer F.Cu) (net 1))
 (segment (start 99.06 132.08) (end 99.6 131.54) (width 0.25) (layer F.Cu) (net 1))
 (segment (start 99.6 131.54) (end 101.6 131.54) (width 0.25) (layer F.Cu) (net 1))
 (segment (start 101.6 131.54) (end 104.14 131.54) (width 0.25) (layer F.Cu) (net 1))
 (segment (start 106.68 129.54) (end 106.68 124.46) (width 0.25) (layer F.Cu) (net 1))
 (segment (start 106.68 124.46) (end 107.22 123.92) (width 0.25) (layer F.Cu) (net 1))
 (segment (start 107.22 123.92) (end 111.76 123.92) (width 0.25) (layer F.Cu) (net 1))
 (segment (start 104.14 131.54) (end 104.68 131.54) (width 0.25) (layer F.Cu) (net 1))
 (segment (start 104.68 131.54) (end 106.68 129.54) (width 0.25) (layer F.Cu) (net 1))
 (segment (start 107.315 137.795) (end 107.061 137.795) (width 0.25) (layer F.Cu) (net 1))
 (segment (start 107.061 137.795) (end 103.251 141.605) (width 0.25) (layer F.Cu) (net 1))
 (segment (start 103.251 141.605) (end 100.965 141.605) (width 0.25) (layer F.Cu) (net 1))
 (segment (start 106.68 129.54) (end 108.204 131.064) (width 0.25) (layer F.Cu) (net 1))
 (segment (start 108.204 131.064) (end 108.204 132.08) (width 0.25) (layer F.Cu) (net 1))
 (segment (start 108.204 132.08) (end 108.204 136.652) (width 0.25) (layer B.Cu) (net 1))
 (segment (start 108.204 136.652) (end 108.204 137.16) (width 0.25) (layer F.Cu) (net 1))
 (segment (start 108.204 137.16) (end 107.95 137.16) (width 0.25) (layer F.Cu) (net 1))
 (segment (start 107.95 137.16) (end 107.315 137.795) (width 0.25) (layer F.Cu) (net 1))
 (segment (start 97.13 132.08) (end 90.83 132.08) (width 0.25) (layer F.Cu) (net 1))
 (via (at 108.204 132.08) (size 0.6) (layers F.Cu B.Cu) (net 1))
 (via (at 108.204 136.652) (size 0.6) (layers F.Cu B.Cu) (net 1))
 (segment (start 99.568 142.748) (end 100.838 142.748) (width 0.25) (layer F.Cu) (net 11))
 (segment (start 100.838 142.748) (end 100.965 142.875) (width 0.25) (layer F.Cu) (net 11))
 (segment (start 99.568 121.412) (end 99.568 142.748) (width 0.25) (layer B.Cu) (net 11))
 (segment (start 99.568 119.206) (end 99.568 121.412) (width 0.25) (layer F.Cu) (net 11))
 (via (at 99.568 142.748) (size 0.6) (layers F.Cu B.Cu) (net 11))
 (via (at 99.568 121.412) (size 0.6) (layers F.Cu B.Cu) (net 11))
 (segment (start 98.552 143.256) (end 99.568 144.272) (width 0.25) (layer F.Cu) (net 10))
 (segment (start 99.568 144.272) (end 100.838 144.272) (width 0.25) (layer F.Cu) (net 10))
 (segment (start 100.838 144.272) (end 100.965 144.145) (width 0.25) (layer F.Cu) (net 10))
 (segment (start 100.218 119.206) (end 100.218 122.794) (width 0.25) (layer F.Cu) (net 10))
 (segment (start 100.218 122.794) (end 100.076 122.936) (width 0.25) (layer F.Cu) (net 10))
 (segment (start 100.076 122.936) (end 98.552 122.936) (width 0.25) (layer F.Cu) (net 10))
 (segment (start 98.552 122.936) (end 98.552 143.256) (width 0.25) (layer B.Cu) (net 10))
 (via (at 98.552 143.256) (size 0.6) (layers F.Cu B.Cu) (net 10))
 (via (at 98.552 122.936) (size 0.6) (layers F.Cu B.Cu) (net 10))
 (segment (start 101.09 157.48) (end 101.09 157.734) (width 0.25) (layer F.Cu) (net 17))
 (segment (start 108.712 151.892) (end 101.092 151.892) (width 0.25) (layer F.Cu) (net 17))
 (segment (start 101.092 151.892) (end 101.092 157.478) (width 0.25) (layer F.Cu) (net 17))
 (segment (start 101.092 157.478) (end 101.09 157.48) (width 0.25) (layer F.Cu) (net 17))
 (segment (start 111.76 125.92) (end 115.38 125.92) (width 0.25) (layer F.Cu) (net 17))
 (segment (start 115.38 125.92) (end 116.84 124.46) (width 0.25) (layer F.Cu) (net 17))
 (segment (start 111.76 125.92) (end 111.696 125.984) (width 0.25) (layer F.Cu) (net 17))
 (segment (start 111.696 125.984) (end 110.236 125.984) (width 0.25) (layer F.Cu) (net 17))
 (segment (start 110.236 125.984) (end 109.22 127) (width 0.25) (layer F.Cu) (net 17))
 (segment (start 109.22 127) (end 109.22 131.064) (width 0.25) (layer F.Cu) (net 17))
 (segment (start 109.22 149.352) (end 109.22 151.384) (width 0.25) (layer B.Cu) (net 17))
 (segment (start 109.22 151.384) (end 108.712 151.892) (width 0.25) (layer B.Cu) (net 17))
 (segment (start 109.22 136.144) (end 109.22 149.352) (width 0.25) (layer F.Cu) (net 17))
 (segment (start 109.22 131.064) (end 109.22 136.144) (width 0.25) (layer B.Cu) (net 17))
 (via (at 108.712 151.892) (size 0.6) (layers F.Cu B.Cu) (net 17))
 (via (at 109.22 149.352) (size 0.6) (layers F.Cu B.Cu) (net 17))
 (via (at 109.22 136.144) (size 0.6) (layers F.Cu B.Cu) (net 17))
 (via (at 109.22 131.064) (size 0.6) (layers F.Cu B.Cu) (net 17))
 (segment (start 99.06 157.48) (end 99.06 157.734) (width 0.25) (layer F.Cu) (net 18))
 (segment (start 110.236 135.636) (end 110.236 150.368) (width 0.25) (layer F.Cu) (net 18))
 (segment (start 110.236 150.368) (end 99.568 150.368) (width 0.25) (layer F.Cu) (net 18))
 (segment (start 99.568 150.368) (end 99.06 150.876) (width 0.25) (layer F.Cu) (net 18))
 (segment (start 99.06 150.876) (end 99.06 157.48) (width 0.25) (layer F.Cu) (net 18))
 (segment (start 116.84 127) (end 112.68 127) (width 0.25) (layer F.Cu) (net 18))
 (segment (start 112.68 127) (end 111.76 127.92) (width 0.25) (layer F.Cu) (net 18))
 (segment (start 110.236 128.016) (end 110.236 135.636) (width 0.25) (layer B.Cu) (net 18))
 (segment (start 111.76 127.92) (end 111.664 128.016) (width 0.25) (layer F.Cu) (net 18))
 (segment (start 111.664 128.016) (end 110.236 128.016) (width 0.25) (layer F.Cu) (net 18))
 (via (at 110.236 128.016) (size 0.6) (layers F.Cu B.Cu) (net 18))
 (via (at 110.236 135.636) (size 0.6) (layers F.Cu B.Cu) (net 18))
 (segment (start 106.426 160.15) (end 106.68 160.404) (width 0.25) (layer F.Cu) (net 19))
 (segment (start 106.426 160.15) (end 93.214 160.15) (width 0.25) (layer F.Cu) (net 19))
 (segment (start 106.68 160.15) (end 106.426 160.15) (width 0.25) (layer F.Cu) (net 19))
 (segment (start 93.214 160.15) (end 92.96 160.404) (width 0.25) (layer F.Cu) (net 19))
 (segment (start 93.214 160.15) (end 92.96 160.15) (width 0.25) (layer F.Cu) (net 19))
 (segment (start 82.042 121.92) (end 85.122 121.92) (width 0.25) (layer F.Cu) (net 20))
 (segment (start 85.122 121.92) (end 87.122 123.92) (width 0.25) (layer F.Cu) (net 20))
 (segment (start 87.122 125.92) (end 83.502 125.92) (width 0.25) (layer F.Cu) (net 21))
 (segment (start 83.502 125.92) (end 82.042 124.46) (width 0.25) (layer F.Cu) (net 21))
 (segment (start 87.122 127.92) (end 82.962 127.92) (width 0.25) (layer F.Cu) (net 22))
 (segment (start 82.962 127.92) (end 82.042 127) (width 0.25) (layer F.Cu) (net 22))
 (segment (start 82.042 129.54) (end 86.742 129.54) (width 0.25) (layer F.Cu) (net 23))
 (segment (start 86.742 129.54) (end 87.122 129.92) (width 0.25) (layer F.Cu) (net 23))
 (segment (start 82.042 132.08) (end 86.962 132.08) (width 0.25) (layer F.Cu) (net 24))
 (segment (start 86.962 132.08) (end 87.122 131.92) (width 0.25) (layer F.Cu) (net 24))
 (segment (start 87.122 133.92) (end 82.742 133.92) (width 0.25) (layer F.Cu) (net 25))
 (segment (start 82.742 133.92) (end 82.042 134.62) (width 0.25) (layer F.Cu) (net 25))
 (segment (start 82.042 137.16) (end 85.882 137.16) (width 0.25) (layer F.Cu) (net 26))
 (segment (start 85.882 137.16) (end 87.122 135.92) (width 0.25) (layer F.Cu) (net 26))
 (segment (start 87.122 137.92) (end 83.822 137.92) (width 0.25) (layer F.Cu) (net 27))
 (segment (start 83.822 137.92) (end 82.042 139.7) (width 0.25) (layer F.Cu) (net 27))
 (segment (start 87.122 139.92) (end 84.362 139.92) (width 0.25) (layer F.Cu) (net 28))
 (segment (start 84.362 139.92) (end 82.042 142.24) (width 0.25) (layer F.Cu) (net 28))
 (segment (start 87.122 141.92) (end 84.902 141.92) (width 0.25) (layer F.Cu) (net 29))
 (segment (start 84.902 141.92) (end 82.042 144.78) (width 0.25) (layer F.Cu) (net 29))
 (segment (start 87.122 143.92) (end 85.442 143.92) (width 0.25) (layer F.Cu) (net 30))
 (segment (start 85.442 143.92) (end 82.042 147.32) (width 0.25) (layer F.Cu) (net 30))
 (segment (start 87.122 145.92) (end 85.982 145.92) (width 0.25) (layer F.Cu) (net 31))
 (segment (start 85.982 145.92) (end 82.042 149.86) (width 0.25) (layer F.Cu) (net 31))
 (segment (start 87.122 147.92) (end 86.522 147.92) (width 0.25) (layer F.Cu) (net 32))
 (segment (start 86.522 147.92) (end 82.042 152.4) (width 0.25) (layer F.Cu) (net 32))
 (segment (start 87.122 149.92) (end 87.062 149.92) (width 0.25) (layer F.Cu) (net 33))
 (segment (start 87.062 149.92) (end 82.042 154.94) (width 0.25) (layer F.Cu) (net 33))
 (segment (start 82.042 157.48) (end 82.042 157) (width 0.25) (layer F.Cu) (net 34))
 (segment (start 82.042 157) (end 87.122 151.92) (width 0.25) (layer F.Cu) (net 34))
 (segment (start 111.76 129.92) (end 111.38 129.92) (width 0.25) (layer F.Cu) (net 13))
 (segment (start 100.965 139.065) (end 102.615 139.065) (width 0.25) (layer F.Cu) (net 13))
 (segment (start 102.615 139.065) (end 111.76 129.92) (width 0.25) (layer F.Cu) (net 13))
 (segment (start 111.76 129.92) (end 116.46 129.92) (width 0.25) (layer F.Cu) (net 13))
 (segment (start 116.46 129.92) (end 116.84 129.54) (width 0.25) (layer F.Cu) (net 13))
 (segment (start 111.76 131.92) (end 116.68 131.92) (width 0.25) (layer F.Cu) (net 12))
 (segment (start 116.68 131.92) (end 116.84 132.08) (width 0.25) (layer F.Cu) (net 12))
 (segment (start 100.965 140.335) (end 101.092 140.208) (width 0.25) (layer F.Cu) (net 12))
 (segment (start 101.092 140.208) (end 103.124 140.208) (width 0.25) (layer F.Cu) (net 12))
 (segment (start 103.124 140.208) (end 111.252 132.08) (width 0.25) (layer F.Cu) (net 12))
 (segment (start 111.252 132.08) (end 111.76 131.92) (width 0.25) (layer F.Cu) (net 12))
 (segment (start 116.84 134.62) (end 112.46 134.62) (width 0.25) (layer F.Cu) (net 35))
 (segment (start 112.46 134.62) (end 111.76 133.92) (width 0.25) (layer F.Cu) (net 35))
 (segment (start 111.76 135.92) (end 115.6 135.92) (width 0.25) (layer F.Cu) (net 36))
 (segment (start 115.6 135.92) (end 116.84 137.16) (width 0.25) (layer F.Cu) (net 36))
 (segment (start 111.76 137.92) (end 115.06 137.92) (width 0.25) (layer F.Cu) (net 37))
 (segment (start 115.06 137.92) (end 116.84 139.7) (width 0.25) (layer F.Cu) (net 37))
 (segment (start 111.76 139.92) (end 114.52 139.92) (width 0.25) (layer F.Cu) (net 38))
 (segment (start 114.52 139.92) (end 116.84 142.24) (width 0.25) (layer F.Cu) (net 38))
 (segment (start 116.84 144.78) (end 114.62 144.78) (width 0.25) (layer F.Cu) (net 39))
 (segment (start 114.62 144.78) (end 111.76 141.92) (width 0.25) (layer F.Cu) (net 39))
 (segment (start 116.84 147.32) (end 115.16 147.32) (width 0.25) (layer F.Cu) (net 40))
 (segment (start 115.16 147.32) (end 111.76 143.92) (width 0.25) (layer F.Cu) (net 40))
 (segment (start 111.76 145.92) (end 112.9 145.92) (width 0.25) (layer F.Cu) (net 41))
 (segment (start 112.9 145.92) (end 116.84 149.86) (width 0.25) (layer F.Cu) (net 41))
 (segment (start 116.84 152.4) (end 116.24 152.4) (width 0.25) (layer F.Cu) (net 42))
 (segment (start 116.24 152.4) (end 111.76 147.92) (width 0.25) (layer F.Cu) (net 42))
 (segment (start 116.84 154.94) (end 116.78 154.94) (width 0.25) (layer F.Cu) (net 43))
 (segment (start 116.78 154.94) (end 111.76 149.92) (width 0.25) (layer F.Cu) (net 43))
 (segment (start 111.76 151.92) (end 111.76 152.4) (width 0.25) (layer F.Cu) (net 44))
 (segment (start 111.76 152.4) (end 116.84 157.48) (width 0.25) (layer F.Cu) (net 44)))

